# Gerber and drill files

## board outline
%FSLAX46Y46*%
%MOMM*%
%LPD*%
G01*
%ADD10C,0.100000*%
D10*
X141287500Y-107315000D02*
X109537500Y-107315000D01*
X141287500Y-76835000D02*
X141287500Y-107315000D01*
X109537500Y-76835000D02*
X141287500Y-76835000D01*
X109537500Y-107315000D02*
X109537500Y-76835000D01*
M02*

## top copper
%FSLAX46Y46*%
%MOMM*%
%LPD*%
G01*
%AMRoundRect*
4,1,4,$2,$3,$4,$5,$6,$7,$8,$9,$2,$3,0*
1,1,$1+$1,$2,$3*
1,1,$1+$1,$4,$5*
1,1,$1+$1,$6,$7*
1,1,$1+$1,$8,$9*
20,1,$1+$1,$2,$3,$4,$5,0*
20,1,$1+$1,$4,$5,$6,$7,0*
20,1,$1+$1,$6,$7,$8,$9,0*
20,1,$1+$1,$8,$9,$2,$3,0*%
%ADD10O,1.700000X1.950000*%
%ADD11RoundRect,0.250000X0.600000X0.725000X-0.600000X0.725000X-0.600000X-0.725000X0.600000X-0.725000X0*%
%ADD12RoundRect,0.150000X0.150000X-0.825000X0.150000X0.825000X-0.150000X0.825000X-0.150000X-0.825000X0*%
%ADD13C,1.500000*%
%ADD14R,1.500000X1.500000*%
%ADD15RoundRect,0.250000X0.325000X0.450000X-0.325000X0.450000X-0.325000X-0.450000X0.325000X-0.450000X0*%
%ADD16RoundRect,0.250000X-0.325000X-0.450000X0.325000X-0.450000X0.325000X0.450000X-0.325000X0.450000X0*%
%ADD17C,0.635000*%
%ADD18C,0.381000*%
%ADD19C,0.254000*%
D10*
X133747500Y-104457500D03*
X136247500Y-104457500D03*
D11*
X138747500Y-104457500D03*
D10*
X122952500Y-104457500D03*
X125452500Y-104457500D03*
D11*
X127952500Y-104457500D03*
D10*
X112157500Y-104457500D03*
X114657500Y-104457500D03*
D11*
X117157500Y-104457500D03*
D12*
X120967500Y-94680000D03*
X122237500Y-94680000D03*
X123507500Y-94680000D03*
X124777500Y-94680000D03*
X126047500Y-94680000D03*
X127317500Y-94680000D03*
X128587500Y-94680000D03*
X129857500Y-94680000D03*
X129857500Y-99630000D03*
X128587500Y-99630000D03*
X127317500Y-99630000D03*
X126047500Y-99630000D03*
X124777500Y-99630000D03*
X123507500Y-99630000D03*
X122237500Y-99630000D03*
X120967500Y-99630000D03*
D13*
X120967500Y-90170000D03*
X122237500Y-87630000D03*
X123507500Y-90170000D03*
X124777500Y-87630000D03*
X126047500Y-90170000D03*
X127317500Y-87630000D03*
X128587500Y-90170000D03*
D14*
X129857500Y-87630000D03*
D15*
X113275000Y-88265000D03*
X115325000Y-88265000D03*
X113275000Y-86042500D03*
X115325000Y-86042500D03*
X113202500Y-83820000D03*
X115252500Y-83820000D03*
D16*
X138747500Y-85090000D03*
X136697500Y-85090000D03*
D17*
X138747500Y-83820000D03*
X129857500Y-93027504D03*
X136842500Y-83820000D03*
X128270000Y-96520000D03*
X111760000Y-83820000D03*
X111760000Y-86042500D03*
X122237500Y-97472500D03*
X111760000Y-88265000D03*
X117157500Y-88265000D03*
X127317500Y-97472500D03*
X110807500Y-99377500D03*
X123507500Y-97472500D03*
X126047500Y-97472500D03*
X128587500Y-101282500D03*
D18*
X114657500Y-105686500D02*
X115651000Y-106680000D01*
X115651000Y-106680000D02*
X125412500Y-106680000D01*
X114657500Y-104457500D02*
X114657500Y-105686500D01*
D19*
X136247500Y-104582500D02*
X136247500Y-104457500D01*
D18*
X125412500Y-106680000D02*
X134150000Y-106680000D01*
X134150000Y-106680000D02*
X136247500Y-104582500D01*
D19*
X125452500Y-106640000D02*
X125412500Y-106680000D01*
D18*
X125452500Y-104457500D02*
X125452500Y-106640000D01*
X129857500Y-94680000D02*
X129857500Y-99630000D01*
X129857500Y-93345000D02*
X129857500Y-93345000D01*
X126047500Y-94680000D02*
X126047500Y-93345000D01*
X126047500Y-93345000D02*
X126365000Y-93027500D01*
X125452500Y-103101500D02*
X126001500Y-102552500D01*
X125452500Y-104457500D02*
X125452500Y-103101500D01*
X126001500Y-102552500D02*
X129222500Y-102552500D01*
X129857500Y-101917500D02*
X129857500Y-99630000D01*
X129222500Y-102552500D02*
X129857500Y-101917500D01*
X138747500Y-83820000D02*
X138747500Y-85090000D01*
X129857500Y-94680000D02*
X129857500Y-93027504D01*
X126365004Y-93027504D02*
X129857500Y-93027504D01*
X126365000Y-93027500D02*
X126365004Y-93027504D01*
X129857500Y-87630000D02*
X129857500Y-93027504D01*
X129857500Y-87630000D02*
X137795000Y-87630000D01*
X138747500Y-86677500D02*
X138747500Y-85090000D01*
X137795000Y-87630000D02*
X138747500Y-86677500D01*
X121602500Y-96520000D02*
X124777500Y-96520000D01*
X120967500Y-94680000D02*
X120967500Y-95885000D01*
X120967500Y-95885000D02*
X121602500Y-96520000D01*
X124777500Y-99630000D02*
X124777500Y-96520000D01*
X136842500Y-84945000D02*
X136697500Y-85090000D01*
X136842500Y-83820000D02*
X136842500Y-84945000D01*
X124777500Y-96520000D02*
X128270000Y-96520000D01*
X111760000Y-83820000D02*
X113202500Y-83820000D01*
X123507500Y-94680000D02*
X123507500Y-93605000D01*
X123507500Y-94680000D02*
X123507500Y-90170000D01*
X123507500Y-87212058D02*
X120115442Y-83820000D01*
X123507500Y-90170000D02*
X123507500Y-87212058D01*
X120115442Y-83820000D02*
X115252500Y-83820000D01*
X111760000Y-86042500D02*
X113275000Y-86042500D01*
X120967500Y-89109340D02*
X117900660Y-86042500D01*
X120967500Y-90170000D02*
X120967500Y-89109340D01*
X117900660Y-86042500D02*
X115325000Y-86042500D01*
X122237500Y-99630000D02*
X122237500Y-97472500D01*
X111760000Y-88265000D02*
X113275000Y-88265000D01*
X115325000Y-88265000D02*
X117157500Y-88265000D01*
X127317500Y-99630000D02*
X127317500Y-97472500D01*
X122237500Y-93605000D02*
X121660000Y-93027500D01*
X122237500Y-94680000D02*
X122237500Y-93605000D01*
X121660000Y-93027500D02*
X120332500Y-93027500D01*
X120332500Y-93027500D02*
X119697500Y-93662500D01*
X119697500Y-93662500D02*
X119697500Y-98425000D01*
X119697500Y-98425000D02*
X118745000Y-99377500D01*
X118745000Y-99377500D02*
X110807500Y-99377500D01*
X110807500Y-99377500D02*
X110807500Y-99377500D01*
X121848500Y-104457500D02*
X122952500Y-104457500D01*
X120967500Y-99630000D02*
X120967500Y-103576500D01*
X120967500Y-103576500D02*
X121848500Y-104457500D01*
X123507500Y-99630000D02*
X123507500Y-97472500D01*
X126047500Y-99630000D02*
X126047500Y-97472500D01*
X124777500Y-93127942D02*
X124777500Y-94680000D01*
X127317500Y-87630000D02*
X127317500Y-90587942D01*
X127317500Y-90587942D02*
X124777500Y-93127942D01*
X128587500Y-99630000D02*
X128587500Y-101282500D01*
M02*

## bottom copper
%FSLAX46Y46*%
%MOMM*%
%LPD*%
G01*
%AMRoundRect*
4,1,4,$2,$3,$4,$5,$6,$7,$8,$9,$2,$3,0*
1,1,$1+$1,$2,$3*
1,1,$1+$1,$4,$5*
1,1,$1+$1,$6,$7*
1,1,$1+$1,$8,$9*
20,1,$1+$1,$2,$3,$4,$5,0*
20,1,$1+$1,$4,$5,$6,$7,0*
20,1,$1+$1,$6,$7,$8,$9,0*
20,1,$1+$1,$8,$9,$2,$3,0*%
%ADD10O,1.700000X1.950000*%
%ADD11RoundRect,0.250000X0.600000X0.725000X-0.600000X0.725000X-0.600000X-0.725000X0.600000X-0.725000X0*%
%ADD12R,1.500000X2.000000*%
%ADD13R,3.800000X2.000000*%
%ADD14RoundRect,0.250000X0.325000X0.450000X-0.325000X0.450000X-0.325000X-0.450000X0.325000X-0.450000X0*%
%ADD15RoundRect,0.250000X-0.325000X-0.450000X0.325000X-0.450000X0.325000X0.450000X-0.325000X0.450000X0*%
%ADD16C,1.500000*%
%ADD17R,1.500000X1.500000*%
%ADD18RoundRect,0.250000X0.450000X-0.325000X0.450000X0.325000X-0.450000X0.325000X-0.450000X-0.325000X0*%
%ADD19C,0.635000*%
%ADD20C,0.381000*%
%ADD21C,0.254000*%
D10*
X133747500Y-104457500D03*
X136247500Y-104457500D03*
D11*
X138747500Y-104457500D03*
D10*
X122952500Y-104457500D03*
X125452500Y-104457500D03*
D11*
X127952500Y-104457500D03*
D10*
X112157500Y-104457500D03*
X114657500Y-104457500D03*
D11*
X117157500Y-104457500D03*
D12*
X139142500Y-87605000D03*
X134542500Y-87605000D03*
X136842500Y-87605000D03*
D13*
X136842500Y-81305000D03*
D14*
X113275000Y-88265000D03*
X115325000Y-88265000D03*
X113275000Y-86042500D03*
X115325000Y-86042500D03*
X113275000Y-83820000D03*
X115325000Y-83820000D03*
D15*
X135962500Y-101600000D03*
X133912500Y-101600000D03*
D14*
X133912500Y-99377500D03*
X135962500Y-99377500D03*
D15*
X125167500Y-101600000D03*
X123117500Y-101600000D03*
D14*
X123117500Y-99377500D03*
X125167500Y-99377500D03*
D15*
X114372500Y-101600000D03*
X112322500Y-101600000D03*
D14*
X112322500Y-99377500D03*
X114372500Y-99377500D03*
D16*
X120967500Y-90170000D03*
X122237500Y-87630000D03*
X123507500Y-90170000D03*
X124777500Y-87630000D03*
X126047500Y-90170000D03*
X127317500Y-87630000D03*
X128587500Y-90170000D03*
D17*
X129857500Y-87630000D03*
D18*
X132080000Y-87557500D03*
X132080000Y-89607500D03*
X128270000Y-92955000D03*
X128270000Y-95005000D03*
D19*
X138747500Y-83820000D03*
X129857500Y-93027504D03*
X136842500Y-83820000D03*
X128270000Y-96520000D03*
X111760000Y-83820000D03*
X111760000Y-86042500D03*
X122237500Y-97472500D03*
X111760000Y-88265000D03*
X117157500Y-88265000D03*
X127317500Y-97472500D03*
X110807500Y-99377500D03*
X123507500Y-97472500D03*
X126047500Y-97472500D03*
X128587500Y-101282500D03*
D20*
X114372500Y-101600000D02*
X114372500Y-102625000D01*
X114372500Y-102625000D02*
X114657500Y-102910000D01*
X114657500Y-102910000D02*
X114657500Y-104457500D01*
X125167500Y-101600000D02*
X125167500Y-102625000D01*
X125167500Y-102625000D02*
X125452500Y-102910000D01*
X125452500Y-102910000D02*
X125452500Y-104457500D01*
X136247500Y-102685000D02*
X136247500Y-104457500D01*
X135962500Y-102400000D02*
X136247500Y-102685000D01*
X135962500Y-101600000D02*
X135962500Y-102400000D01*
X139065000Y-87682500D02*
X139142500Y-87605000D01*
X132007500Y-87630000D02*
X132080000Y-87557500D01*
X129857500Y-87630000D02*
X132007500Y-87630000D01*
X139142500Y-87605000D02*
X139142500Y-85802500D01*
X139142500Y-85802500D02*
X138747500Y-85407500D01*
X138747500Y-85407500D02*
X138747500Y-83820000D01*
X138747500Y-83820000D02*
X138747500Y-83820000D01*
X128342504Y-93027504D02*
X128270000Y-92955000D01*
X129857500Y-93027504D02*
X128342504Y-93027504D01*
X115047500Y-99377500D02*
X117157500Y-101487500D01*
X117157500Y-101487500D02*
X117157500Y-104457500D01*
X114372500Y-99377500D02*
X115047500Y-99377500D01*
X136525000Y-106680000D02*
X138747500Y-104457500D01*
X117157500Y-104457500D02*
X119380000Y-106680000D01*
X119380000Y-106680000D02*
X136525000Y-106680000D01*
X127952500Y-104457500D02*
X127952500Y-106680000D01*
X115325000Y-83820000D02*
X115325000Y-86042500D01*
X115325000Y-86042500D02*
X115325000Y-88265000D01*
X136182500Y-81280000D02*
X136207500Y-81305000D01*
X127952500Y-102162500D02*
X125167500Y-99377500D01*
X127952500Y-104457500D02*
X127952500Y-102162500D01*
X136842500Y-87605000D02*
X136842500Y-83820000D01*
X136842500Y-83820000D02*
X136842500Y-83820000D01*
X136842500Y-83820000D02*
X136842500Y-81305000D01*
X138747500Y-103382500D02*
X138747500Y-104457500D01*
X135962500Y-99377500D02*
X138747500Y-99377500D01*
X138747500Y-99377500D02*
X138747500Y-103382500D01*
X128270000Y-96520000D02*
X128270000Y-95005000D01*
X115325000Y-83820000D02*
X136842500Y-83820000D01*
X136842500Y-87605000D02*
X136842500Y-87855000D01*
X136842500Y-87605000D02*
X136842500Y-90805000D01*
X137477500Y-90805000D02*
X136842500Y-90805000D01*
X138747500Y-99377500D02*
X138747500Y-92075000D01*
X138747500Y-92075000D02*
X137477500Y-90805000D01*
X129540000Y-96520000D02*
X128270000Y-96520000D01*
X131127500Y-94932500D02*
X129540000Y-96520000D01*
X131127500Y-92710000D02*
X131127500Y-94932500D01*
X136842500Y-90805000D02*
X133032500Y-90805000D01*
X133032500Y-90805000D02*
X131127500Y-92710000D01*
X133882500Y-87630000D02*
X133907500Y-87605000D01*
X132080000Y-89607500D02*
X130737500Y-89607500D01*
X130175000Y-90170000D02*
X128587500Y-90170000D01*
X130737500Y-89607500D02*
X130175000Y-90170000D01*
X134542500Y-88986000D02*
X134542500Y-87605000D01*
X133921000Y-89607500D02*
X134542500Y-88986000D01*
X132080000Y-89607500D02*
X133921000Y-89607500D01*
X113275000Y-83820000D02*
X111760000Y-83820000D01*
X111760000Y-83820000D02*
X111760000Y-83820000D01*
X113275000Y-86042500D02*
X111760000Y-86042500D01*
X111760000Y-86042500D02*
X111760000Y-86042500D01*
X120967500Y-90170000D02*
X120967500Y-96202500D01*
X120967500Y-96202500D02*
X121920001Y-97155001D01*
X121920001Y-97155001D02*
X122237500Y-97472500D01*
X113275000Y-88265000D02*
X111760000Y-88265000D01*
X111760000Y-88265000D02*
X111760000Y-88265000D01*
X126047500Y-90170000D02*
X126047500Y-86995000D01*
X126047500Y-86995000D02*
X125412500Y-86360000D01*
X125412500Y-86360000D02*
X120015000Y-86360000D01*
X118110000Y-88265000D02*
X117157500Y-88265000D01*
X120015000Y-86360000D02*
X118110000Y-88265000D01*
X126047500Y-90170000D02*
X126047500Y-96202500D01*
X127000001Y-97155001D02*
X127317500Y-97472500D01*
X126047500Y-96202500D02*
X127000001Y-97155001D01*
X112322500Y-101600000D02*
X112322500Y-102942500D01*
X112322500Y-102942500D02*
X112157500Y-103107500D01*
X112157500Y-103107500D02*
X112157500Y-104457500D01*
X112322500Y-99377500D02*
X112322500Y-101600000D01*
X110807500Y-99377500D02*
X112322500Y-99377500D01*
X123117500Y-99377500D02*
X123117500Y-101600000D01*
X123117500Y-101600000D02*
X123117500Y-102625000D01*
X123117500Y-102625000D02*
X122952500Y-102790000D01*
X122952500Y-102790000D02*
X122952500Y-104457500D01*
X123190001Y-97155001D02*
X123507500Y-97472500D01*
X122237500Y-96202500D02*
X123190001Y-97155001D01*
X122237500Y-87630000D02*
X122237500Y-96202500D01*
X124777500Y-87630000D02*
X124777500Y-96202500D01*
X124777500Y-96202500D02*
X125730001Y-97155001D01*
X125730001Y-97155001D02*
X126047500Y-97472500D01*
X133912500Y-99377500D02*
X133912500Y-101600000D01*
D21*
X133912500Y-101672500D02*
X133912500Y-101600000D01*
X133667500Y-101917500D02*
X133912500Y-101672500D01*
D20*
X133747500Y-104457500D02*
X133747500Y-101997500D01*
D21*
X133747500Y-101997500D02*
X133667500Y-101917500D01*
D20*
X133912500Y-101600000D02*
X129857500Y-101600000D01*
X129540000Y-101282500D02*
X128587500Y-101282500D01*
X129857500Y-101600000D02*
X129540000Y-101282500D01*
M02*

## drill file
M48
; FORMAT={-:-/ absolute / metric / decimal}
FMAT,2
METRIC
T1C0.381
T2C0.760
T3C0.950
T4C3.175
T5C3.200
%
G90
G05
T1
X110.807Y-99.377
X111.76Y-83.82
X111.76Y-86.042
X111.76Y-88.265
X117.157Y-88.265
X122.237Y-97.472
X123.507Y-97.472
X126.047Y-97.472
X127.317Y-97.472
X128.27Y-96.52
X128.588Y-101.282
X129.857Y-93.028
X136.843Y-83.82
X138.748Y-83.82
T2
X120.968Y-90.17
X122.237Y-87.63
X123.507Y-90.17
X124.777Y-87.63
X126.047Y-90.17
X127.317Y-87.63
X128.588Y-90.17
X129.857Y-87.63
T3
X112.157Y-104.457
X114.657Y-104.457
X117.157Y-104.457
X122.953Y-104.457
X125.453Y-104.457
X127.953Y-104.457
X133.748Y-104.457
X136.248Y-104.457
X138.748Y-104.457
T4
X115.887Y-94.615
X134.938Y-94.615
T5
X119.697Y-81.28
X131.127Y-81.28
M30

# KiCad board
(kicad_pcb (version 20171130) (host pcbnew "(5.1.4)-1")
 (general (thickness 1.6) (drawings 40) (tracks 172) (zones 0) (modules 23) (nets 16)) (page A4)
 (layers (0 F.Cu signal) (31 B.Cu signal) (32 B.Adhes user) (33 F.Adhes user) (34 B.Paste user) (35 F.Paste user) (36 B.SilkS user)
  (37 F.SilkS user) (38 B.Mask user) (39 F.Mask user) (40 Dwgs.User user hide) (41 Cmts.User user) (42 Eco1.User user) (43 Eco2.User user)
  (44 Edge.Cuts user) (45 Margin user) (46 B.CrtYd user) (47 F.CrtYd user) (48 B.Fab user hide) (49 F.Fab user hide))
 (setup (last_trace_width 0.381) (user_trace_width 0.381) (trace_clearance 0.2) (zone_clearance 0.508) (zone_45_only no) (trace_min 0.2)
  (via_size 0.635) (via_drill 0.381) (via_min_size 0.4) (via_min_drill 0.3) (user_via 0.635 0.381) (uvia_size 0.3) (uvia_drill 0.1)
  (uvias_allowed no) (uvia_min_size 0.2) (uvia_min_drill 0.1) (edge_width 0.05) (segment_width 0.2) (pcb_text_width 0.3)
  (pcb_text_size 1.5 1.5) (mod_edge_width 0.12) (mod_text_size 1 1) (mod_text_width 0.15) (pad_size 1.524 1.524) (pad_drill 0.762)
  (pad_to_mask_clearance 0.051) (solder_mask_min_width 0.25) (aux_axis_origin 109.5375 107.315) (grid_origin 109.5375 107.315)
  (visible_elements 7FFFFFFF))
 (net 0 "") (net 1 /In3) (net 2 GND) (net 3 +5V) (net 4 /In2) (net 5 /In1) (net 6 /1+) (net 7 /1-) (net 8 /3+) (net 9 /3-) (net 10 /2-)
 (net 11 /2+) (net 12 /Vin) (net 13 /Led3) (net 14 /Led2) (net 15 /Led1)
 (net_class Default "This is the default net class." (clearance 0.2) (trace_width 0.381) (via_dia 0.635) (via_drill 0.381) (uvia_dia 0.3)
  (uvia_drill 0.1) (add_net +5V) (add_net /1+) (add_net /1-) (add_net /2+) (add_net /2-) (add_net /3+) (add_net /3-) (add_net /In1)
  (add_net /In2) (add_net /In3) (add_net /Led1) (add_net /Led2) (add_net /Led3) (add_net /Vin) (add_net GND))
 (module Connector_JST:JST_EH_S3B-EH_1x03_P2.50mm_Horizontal (layer F.Cu) (at 138.7475 104.4575 180)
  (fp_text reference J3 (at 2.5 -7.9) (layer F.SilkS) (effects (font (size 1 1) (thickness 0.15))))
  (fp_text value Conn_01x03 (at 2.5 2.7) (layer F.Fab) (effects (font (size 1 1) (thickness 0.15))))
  (pad 3 thru_hole oval (at 5 0 180) (size 1.7 1.95) (drill 0.95) (layers *.Cu *.Mask) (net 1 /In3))
  (pad 2 thru_hole oval (at 2.5 0 180) (size 1.7 1.95) (drill 0.95) (layers *.Cu *.Mask) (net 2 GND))
  (pad 1 thru_hole roundrect (at 0 0 180) (size 1.7 1.95) (drill 0.95) (layers *.Cu *.Mask) (roundrect_rratio 0.147059) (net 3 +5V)))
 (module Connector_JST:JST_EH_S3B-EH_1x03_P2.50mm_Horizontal (layer F.Cu) (at 127.9525 104.4575 180)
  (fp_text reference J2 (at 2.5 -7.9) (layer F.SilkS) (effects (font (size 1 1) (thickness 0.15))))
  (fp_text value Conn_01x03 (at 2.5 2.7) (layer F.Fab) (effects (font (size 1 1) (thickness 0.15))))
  (pad 3 thru_hole oval (at 5 0 180) (size 1.7 1.95) (drill 0.95) (layers *.Cu *.Mask) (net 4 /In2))
  (pad 2 thru_hole oval (at 2.5 0 180) (size 1.7 1.95) (drill 0.95) (layers *.Cu *.Mask) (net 2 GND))
  (pad 1 thru_hole roundrect (at 0 0 180) (size 1.7 1.95) (drill 0.95) (layers *.Cu *.Mask) (roundrect_rratio 0.147059) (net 3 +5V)))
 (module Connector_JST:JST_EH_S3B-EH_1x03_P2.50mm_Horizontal (layer F.Cu) (at 117.1575 104.4575 180)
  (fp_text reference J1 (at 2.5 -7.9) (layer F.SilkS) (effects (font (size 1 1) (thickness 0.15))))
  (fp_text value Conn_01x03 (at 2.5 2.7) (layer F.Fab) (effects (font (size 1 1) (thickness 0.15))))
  (pad 3 thru_hole oval (at 5 0 180) (size 1.7 1.95) (drill 0.95) (layers *.Cu *.Mask) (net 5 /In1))
  (pad 2 thru_hole oval (at 2.5 0 180) (size 1.7 1.95) (drill 0.95) (layers *.Cu *.Mask) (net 2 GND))
  (pad 1 thru_hole roundrect (at 0 0 180) (size 1.7 1.95) (drill 0.95) (layers *.Cu *.Mask) (roundrect_rratio 0.147059) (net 3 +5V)))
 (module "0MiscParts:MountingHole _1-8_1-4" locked (layer F.Cu) (at 134.9375 94.615)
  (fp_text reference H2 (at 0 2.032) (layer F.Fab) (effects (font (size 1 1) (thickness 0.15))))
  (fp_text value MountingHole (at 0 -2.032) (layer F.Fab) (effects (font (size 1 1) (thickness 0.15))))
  (pad "" np_thru_hole circle (at 0 0) (size 3.175 3.175) (drill 3.175) (layers *.Cu *.Mask)))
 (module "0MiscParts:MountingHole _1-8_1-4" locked (layer F.Cu) (at 115.8875 94.615)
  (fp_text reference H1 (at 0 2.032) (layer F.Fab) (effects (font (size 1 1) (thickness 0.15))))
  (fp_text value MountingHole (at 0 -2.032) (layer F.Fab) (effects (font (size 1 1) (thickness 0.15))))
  (pad "" np_thru_hole circle (at 0 0) (size 3.175 3.175) (drill 3.175) (layers *.Cu *.Mask)))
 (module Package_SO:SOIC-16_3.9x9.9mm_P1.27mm (layer F.Cu) (at 125.4125 97.155 90)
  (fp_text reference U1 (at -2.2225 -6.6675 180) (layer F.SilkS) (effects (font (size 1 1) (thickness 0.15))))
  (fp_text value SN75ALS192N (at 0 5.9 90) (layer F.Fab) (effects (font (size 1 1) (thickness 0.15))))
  (pad 16 smd roundrect (at 2.475 -4.445 90) (size 1.95 0.6) (layers F.Cu F.Paste F.Mask) (roundrect_rratio 0.25) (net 3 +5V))
  (pad 15 smd roundrect (at 2.475 -3.175 90) (size 1.95 0.6) (layers F.Cu F.Paste F.Mask) (roundrect_rratio 0.25) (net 5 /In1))
  (pad 14 smd roundrect (at 2.475 -1.905 90) (size 1.95 0.6) (layers F.Cu F.Paste F.Mask) (roundrect_rratio 0.25) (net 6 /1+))
  (pad 13 smd roundrect (at 2.475 -0.635 90) (size 1.95 0.6) (layers F.Cu F.Paste F.Mask) (roundrect_rratio 0.25) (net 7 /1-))
  (pad 12 smd roundrect (at 2.475 0.635 90) (size 1.95 0.6) (layers F.Cu F.Paste F.Mask) (roundrect_rratio 0.25) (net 2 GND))
  (pad 11 smd roundrect (at 2.475 1.905 90) (size 1.95 0.6) (layers F.Cu F.Paste F.Mask) (roundrect_rratio 0.25))
  (pad 10 smd roundrect (at 2.475 3.175 90) (size 1.95 0.6) (layers F.Cu F.Paste F.Mask) (roundrect_rratio 0.25))
  (pad 9 smd roundrect (at 2.475 4.445 90) (size 1.95 0.6) (layers F.Cu F.Paste F.Mask) (roundrect_rratio 0.25) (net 2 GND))
  (pad 8 smd roundrect (at -2.475 4.445 90) (size 1.95 0.6) (layers F.Cu F.Paste F.Mask) (roundrect_rratio 0.25) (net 2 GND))
  (pad 7 smd roundrect (at -2.475 3.175 90) (size 1.95 0.6) (layers F.Cu F.Paste F.Mask) (roundrect_rratio 0.25) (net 1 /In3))
  (pad 6 smd roundrect (at -2.475 1.905 90) (size 1.95 0.6) (layers F.Cu F.Paste F.Mask) (roundrect_rratio 0.25) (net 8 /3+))
  (pad 5 smd roundrect (at -2.475 0.635 90) (size 1.95 0.6) (layers F.Cu F.Paste F.Mask) (roundrect_rratio 0.25) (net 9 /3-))
  (pad 4 smd roundrect (at -2.475 -0.635 90) (size 1.95 0.6) (layers F.Cu F.Paste F.Mask) (roundrect_rratio 0.25) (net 3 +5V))
  (pad 3 smd roundrect (at -2.475 -1.905 90) (size 1.95 0.6) (layers F.Cu F.Paste F.Mask) (roundrect_rratio 0.25) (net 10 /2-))
  (pad 2 smd roundrect (at -2.475 -3.175 90) (size 1.95 0.6) (layers F.Cu F.Paste F.Mask) (roundrect_rratio 0.25) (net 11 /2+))
  (pad 1 smd roundrect (at -2.475 -4.445 90) (size 1.95 0.6) (layers F.Cu F.Paste F.Mask) (roundrect_rratio 0.25) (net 4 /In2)))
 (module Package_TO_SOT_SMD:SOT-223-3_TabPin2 (layer B.Cu) (at 136.8425 84.455 90)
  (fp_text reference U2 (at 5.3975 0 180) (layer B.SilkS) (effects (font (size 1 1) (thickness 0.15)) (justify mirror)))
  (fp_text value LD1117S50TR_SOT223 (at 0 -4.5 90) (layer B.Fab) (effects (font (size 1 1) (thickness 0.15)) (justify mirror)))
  (pad 1 smd rect (at -3.15 2.3 90) (size 2 1.5) (layers B.Cu B.Paste B.Mask) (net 2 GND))
  (pad 3 smd rect (at -3.15 -2.3 90) (size 2 1.5) (layers B.Cu B.Paste B.Mask) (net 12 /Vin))
  (pad 2 smd rect (at -3.15 0 90) (size 2 1.5) (layers B.Cu B.Paste B.Mask) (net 3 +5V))
  (pad 2 smd rect (at 3.15 0 90) (size 2 3.8) (layers B.Cu B.Paste B.Mask) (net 3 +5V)))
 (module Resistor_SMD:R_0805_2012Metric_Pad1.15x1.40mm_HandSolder (layer B.Cu) (at 114.3 88.265 180)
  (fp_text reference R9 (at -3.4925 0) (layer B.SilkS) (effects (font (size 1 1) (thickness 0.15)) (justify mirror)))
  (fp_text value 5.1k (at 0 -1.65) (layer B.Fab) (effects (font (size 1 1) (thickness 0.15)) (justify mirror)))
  (pad 2 smd roundrect (at 1.025 0 180) (size 1.15 1.4) (layers B.Cu B.Paste B.Mask) (roundrect_rratio 0.217391) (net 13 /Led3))
  (pad 1 smd roundrect (at -1.025 0 180) (size 1.15 1.4) (layers B.Cu B.Paste B.Mask) (roundrect_rratio 0.217391) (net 3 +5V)))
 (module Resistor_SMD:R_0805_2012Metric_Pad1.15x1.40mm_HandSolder (layer B.Cu) (at 114.3 86.0425 180)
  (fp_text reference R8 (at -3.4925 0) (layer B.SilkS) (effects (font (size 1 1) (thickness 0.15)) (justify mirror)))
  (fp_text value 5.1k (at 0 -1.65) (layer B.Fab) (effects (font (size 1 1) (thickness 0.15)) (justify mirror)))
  (pad 2 smd roundrect (at 1.025 0 180) (size 1.15 1.4) (layers B.Cu B.Paste B.Mask) (roundrect_rratio 0.217391) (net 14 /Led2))
  (pad 1 smd roundrect (at -1.025 0 180) (size 1.15 1.4) (layers B.Cu B.Paste B.Mask) (roundrect_rratio 0.217391) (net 3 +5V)))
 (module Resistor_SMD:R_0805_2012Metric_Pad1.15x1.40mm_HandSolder (layer B.Cu) (at 114.3 83.82 180)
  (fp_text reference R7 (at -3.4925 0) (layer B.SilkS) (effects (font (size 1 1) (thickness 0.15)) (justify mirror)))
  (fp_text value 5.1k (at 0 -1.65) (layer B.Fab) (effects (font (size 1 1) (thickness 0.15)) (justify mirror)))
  (pad 2 smd roundrect (at 1.025 0 180) (size 1.15 1.4) (layers B.Cu B.Paste B.Mask) (roundrect_rratio 0.217391) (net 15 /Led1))
  (pad 1 smd roundrect (at -1.025 0 180) (size 1.15 1.4) (layers B.Cu B.Paste B.Mask) (roundrect_rratio 0.217391) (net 3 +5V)))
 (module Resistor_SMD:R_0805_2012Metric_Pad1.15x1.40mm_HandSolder (layer B.Cu) (at 134.9375 101.6)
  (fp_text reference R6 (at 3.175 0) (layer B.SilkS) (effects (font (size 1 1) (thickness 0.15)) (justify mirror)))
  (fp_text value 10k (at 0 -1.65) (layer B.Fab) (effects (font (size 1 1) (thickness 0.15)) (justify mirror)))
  (pad 2 smd roundrect (at 1.025 0) (size 1.15 1.4) (layers B.Cu B.Paste B.Mask) (roundrect_rratio 0.217391) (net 2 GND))
  (pad 1 smd roundrect (at -1.025 0) (size 1.15 1.4) (layers B.Cu B.Paste B.Mask) (roundrect_rratio 0.217391) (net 1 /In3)))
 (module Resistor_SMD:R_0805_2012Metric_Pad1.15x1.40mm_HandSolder (layer B.Cu) (at 134.9375 99.3775 180)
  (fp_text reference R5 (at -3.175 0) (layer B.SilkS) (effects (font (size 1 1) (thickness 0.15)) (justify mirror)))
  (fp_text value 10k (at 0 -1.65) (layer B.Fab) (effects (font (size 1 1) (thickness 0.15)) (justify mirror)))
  (pad 2 smd roundrect (at 1.025 0 180) (size 1.15 1.4) (layers B.Cu B.Paste B.Mask) (roundrect_rratio 0.217391) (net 1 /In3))
  (pad 1 smd roundrect (at -1.025 0 180) (size 1.15 1.4) (layers B.Cu B.Paste B.Mask) (roundrect_rratio 0.217391) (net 3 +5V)))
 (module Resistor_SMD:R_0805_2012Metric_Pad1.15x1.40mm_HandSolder (layer B.Cu) (at 124.1425 101.6)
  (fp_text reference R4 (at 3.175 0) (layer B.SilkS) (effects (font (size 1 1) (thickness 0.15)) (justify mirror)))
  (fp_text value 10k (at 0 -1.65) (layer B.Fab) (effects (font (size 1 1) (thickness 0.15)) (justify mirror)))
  (pad 2 smd roundrect (at 1.025 0) (size 1.15 1.4) (layers B.Cu B.Paste B.Mask) (roundrect_rratio 0.217391) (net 2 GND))
  (pad 1 smd roundrect (at -1.025 0) (size 1.15 1.4) (layers B.Cu B.Paste B.Mask) (roundrect_rratio 0.217391) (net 4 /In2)))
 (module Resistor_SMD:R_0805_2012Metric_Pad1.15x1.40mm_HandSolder (layer B.Cu) (at 124.1425 99.3775 180)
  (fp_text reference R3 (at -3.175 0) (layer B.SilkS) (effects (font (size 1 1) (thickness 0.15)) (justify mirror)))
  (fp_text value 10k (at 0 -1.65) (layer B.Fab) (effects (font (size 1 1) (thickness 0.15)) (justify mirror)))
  (pad 2 smd roundrect (at 1.025 0 180) (size 1.15 1.4) (layers B.Cu B.Paste B.Mask) (roundrect_rratio 0.217391) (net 4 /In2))
  (pad 1 smd roundrect (at -1.025 0 180) (size 1.15 1.4) (layers B.Cu B.Paste B.Mask) (roundrect_rratio 0.217391) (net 3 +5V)))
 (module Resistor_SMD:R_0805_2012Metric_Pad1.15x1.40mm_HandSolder (layer B.Cu) (at 113.3475 101.6)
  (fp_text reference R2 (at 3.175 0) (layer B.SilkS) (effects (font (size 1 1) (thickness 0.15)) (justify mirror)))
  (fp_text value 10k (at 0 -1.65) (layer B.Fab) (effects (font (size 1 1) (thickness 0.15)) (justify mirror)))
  (pad 2 smd roundrect (at 1.025 0) (size 1.15 1.4) (layers B.Cu B.Paste B.Mask) (roundrect_rratio 0.217391) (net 2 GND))
  (pad 1 smd roundrect (at -1.025 0) (size 1.15 1.4) (layers B.Cu B.Paste B.Mask) (roundrect_rratio 0.217391) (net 5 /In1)))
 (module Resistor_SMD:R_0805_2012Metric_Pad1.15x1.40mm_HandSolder (layer B.Cu) (at 113.3475 99.3775 180)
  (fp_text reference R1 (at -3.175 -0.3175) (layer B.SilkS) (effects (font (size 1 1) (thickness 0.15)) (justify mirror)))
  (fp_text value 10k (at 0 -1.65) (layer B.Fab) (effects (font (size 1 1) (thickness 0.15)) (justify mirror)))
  (pad 2 smd roundrect (at 1.025 0 180) (size 1.15 1.4) (layers B.Cu B.Paste B.Mask) (roundrect_rratio 0.217391) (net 5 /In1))
  (pad 1 smd roundrect (at -1.025 0 180) (size 1.15 1.4) (layers B.Cu B.Paste B.Mask) (roundrect_rratio 0.217391) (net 3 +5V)))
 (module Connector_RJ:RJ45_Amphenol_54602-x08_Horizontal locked (layer F.Cu) (at 129.8575 87.63 180)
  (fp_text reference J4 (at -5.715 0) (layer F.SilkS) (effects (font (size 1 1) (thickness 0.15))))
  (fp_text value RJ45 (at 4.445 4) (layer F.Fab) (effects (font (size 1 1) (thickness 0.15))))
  (pad 8 thru_hole circle (at 8.89 -2.54 180) (size 1.5 1.5) (drill 0.76) (layers *.Cu *.Mask) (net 11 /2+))
  (pad 7 thru_hole circle (at 7.62 0 180) (size 1.5 1.5) (drill 0.76) (layers *.Cu *.Mask) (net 10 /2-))
  (pad 6 thru_hole circle (at 6.35 -2.54 180) (size 1.5 1.5) (drill 0.76) (layers *.Cu *.Mask) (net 6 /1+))
  (pad 5 thru_hole circle (at 5.08 0 180) (size 1.5 1.5) (drill 0.76) (layers *.Cu *.Mask) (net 9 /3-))
  (pad 4 thru_hole circle (at 3.81 -2.54 180) (size 1.5 1.5) (drill 0.76) (layers *.Cu *.Mask) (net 8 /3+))
  (pad 3 thru_hole circle (at 2.54 0 180) (size 1.5 1.5) (drill 0.76) (layers *.Cu *.Mask) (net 7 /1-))
  (pad 2 thru_hole circle (at 1.27 -2.54 180) (size 1.5 1.5) (drill 0.76) (layers *.Cu *.Mask) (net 12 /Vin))
  (pad 1 thru_hole rect (at 0 0 180) (size 1.5 1.5) (drill 0.76) (layers *.Cu *.Mask) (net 2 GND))
  (pad "" np_thru_hole circle (at -1.27 6.35 180) (size 3.2 3.2) (drill 3.2) (layers *.Cu *.Mask))
  (pad "" np_thru_hole circle (at 10.16 6.35 180) (size 3.2 3.2) (drill 3.2) (layers *.Cu *.Mask)))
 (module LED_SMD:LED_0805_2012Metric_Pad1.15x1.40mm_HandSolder (layer F.Cu) (at 114.3 88.265 180)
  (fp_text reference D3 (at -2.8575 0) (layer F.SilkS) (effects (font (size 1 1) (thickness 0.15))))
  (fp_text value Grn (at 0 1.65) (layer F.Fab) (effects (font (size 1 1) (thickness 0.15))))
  (pad 2 smd roundrect (at 1.025 0 180) (size 1.15 1.4) (layers F.Cu F.Paste F.Mask) (roundrect_rratio 0.217391) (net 13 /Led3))
  (pad 1 smd roundrect (at -1.025 0 180) (size 1.15 1.4) (layers F.Cu F.Paste F.Mask) (roundrect_rratio 0.217391) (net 8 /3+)))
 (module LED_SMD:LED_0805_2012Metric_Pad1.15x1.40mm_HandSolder (layer F.Cu) (at 114.3 86.0425 180)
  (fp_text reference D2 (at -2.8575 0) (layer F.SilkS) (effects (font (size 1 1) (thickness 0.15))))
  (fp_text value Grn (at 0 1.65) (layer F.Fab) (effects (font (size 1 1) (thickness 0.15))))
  (pad 2 smd roundrect (at 1.025 0 180) (size 1.15 1.4) (layers F.Cu F.Paste F.Mask) (roundrect_rratio 0.217391) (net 14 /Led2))
  (pad 1 smd roundrect (at -1.025 0 180) (size 1.15 1.4) (layers F.Cu F.Paste F.Mask) (roundrect_rratio 0.217391) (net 11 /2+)))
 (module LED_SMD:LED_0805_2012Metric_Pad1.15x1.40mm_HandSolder (layer F.Cu) (at 114.2275 83.82 180)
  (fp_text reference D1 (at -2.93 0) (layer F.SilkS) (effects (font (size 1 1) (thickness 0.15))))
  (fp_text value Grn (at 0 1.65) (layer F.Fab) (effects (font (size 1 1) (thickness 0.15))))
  (pad 2 smd roundrect (at 1.025 0 180) (size 1.15 1.4) (layers F.Cu F.Paste F.Mask) (roundrect_rratio 0.217391) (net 15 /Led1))
  (pad 1 smd roundrect (at -1.025 0 180) (size 1.15 1.4) (layers F.Cu F.Paste F.Mask) (roundrect_rratio 0.217391) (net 6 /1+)))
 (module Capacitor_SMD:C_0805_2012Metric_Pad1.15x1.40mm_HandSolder (layer F.Cu) (at 137.7225 85.09)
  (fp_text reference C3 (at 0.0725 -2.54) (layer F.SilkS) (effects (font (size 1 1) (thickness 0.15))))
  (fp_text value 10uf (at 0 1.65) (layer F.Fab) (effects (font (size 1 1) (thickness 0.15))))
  (pad 2 smd roundrect (at 1.025 0) (size 1.15 1.4) (layers F.Cu F.Paste F.Mask) (roundrect_rratio 0.217391) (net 2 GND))
  (pad 1 smd roundrect (at -1.025 0) (size 1.15 1.4) (layers F.Cu F.Paste F.Mask) (roundrect_rratio 0.217391) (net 3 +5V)))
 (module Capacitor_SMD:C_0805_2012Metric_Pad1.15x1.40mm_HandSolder (layer B.Cu) (at 132.08 88.5825 90)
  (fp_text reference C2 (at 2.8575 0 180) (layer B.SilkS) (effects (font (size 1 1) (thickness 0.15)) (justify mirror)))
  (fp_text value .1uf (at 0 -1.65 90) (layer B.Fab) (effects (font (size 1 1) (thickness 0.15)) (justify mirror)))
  (pad 2 smd roundrect (at 1.025 0 90) (size 1.15 1.4) (layers B.Cu B.Paste B.Mask) (roundrect_rratio 0.217391) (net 2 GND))
  (pad 1 smd roundrect (at -1.025 0 90) (size 1.15 1.4) (layers B.Cu B.Paste B.Mask) (roundrect_rratio 0.217391) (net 12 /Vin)))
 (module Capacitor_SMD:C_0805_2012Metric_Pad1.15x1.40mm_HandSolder (layer B.Cu) (at 128.27 93.98 90)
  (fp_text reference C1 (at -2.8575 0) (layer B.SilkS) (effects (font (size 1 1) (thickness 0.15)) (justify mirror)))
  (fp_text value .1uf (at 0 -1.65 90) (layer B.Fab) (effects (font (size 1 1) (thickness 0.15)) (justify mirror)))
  (pad 2 smd roundrect (at 1.025 0 90) (size 1.15 1.4) (layers B.Cu B.Paste B.Mask) (roundrect_rratio 0.217391) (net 2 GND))
  (pad 1 smd roundrect (at -1.025 0 90) (size 1.15 1.4) (layers B.Cu B.Paste B.Mask) (roundrect_rratio 0.217391) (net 3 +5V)))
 (gr_line (start 141.2875 107.315) (end 109.5375 107.315) (layer Edge.Cuts) (width 0.1))
 (gr_line (start 141.2875 76.835) (end 141.2875 107.315) (layer Edge.Cuts) (width 0.1))
 (gr_line (start 109.5375 76.835) (end 141.2875 76.835) (layer Edge.Cuts) (width 0.1))
 (gr_line (start 109.5375 107.315) (end 109.5375 76.835) (layer Edge.Cuts) (width 0.1))
 (segment (start 114.3725 101.6) (end 114.3725 102.625) (width 0.381) (layer B.Cu) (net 2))
 (segment (start 114.3725 102.625) (end 114.6575 102.91) (width 0.381) (layer B.Cu) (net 2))
 (segment (start 114.6575 102.91) (end 114.6575 104.4575) (width 0.381) (layer B.Cu) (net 2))
 (segment (start 125.1675 101.6) (end 125.1675 102.625) (width 0.381) (layer B.Cu) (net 2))
 (segment (start 125.1675 102.625) (end 125.4525 102.91) (width 0.381) (layer B.Cu) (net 2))
 (segment (start 125.4525 102.91) (end 125.4525 104.4575) (width 0.381) (layer B.Cu) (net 2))
 (segment (start 136.2475 102.685) (end 136.2475 104.4575) (width 0.381) (layer B.Cu) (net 2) (status 1000000))
 (segment (start 135.9625 102.4) (end 136.2475 102.685) (width 0.381) (layer B.Cu) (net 2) (status 1000000))
 (segment (start 135.9625 101.6) (end 135.9625 102.4) (width 0.381) (layer B.Cu) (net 2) (status 1000000))
 (segment (start 114.6575 105.6865) (end 115.651 106.68) (width 0.381) (layer F.Cu) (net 2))
 (segment (start 115.651 106.68) (end 125.4125 106.68) (width 0.381) (layer F.Cu) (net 2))
 (segment (start 114.6575 104.4575) (end 114.6575 105.6865) (width 0.381) (layer F.Cu) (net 2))
 (segment (start 136.2475 104.5825) (end 136.2475 104.4575) (width 0.254) (layer F.Cu) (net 2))
 (segment (start 125.4125 106.68) (end 134.15 106.68) (width 0.381) (layer F.Cu) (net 2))
 (segment (start 134.15 106.68) (end 136.2475 104.5825) (width 0.381) (layer F.Cu) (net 2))
 (segment (start 125.4525 106.64) (end 125.4125 106.68) (width 0.254) (layer F.Cu) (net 2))
 (segment (start 125.4525 104.4575) (end 125.4525 106.64) (width 0.381) (layer F.Cu) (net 2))
 (segment (start 129.8575 94.68) (end 129.8575 99.63) (width 0.381) (layer F.Cu) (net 2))
 (segment (start 129.8575 93.345) (end 129.8575 93.345) (width 0.381) (layer F.Cu) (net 2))
 (segment (start 126.0475 94.68) (end 126.0475 93.345) (width 0.381) (layer F.Cu) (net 2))
 (segment (start 126.0475 93.345) (end 126.365 93.0275) (width 0.381) (layer F.Cu) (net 2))
 (segment (start 125.4525 103.1015) (end 126.0015 102.5525) (width 0.381) (layer F.Cu) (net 2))
 (segment (start 125.4525 104.4575) (end 125.4525 103.1015) (width 0.381) (layer F.Cu) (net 2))
 (segment (start 126.0015 102.5525) (end 129.2225 102.5525) (width 0.381) (layer F.Cu) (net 2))
 (segment (start 129.8575 101.9175) (end 129.8575 99.63) (width 0.381) (layer F.Cu) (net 2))
 (segment (start 129.2225 102.5525) (end 129.8575 101.9175) (width 0.381) (layer F.Cu) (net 2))
 (segment (start 139.065 87.6825) (end 139.1425 87.605) (width 0.381) (layer B.Cu) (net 2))
 (segment (start 132.0075 87.63) (end 132.08 87.5575) (width 0.381) (layer B.Cu) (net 2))
 (segment (start 129.8575 87.63) (end 132.0075 87.63) (width 0.381) (layer B.Cu) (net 2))
 (segment (start 139.1425 87.605) (end 139.1425 85.8025) (width 0.381) (layer B.Cu) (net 2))
 (segment (start 139.1425 85.8025) (end 138.7475 85.4075) (width 0.381) (layer B.Cu) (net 2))
 (segment (start 138.7475 85.4075) (end 138.7475 83.82) (width 0.381) (layer B.Cu) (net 2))
 (segment (start 138.7475 83.82) (end 138.7475 83.82) (width 0.381) (layer B.Cu) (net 2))
 (via (at 138.7475 83.82) (size 0.635) (drill 0.381) (layers F.Cu B.Cu) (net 2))
 (segment (start 138.7475 83.82) (end 138.7475 85.09) (width 0.381) (layer F.Cu) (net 2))
 (via (at 129.8575 93.027504) (size 0.635) (drill 0.381) (layers F.Cu B.Cu) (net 2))
 (segment (start 129.8575 94.68) (end 129.8575 93.027504) (width 0.381) (layer F.Cu) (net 2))
 (segment (start 126.365004 93.027504) (end 129.8575 93.027504) (width 0.381) (layer F.Cu) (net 2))
 (segment (start 126.365 93.0275) (end 126.365004 93.027504) (width 0.381) (layer F.Cu) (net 2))
 (segment (start 129.8575 87.63) (end 129.8575 93.027504) (width 0.381) (layer F.Cu) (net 2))
 (segment (start 128.342504 93.027504) (end 128.27 92.955) (width 0.381) (layer B.Cu) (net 2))
 (segment (start 129.8575 93.027504) (end 128.342504 93.027504) (width 0.381) (layer B.Cu) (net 2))
 (segment (start 129.8575 87.63) (end 137.795 87.63) (width 0.381) (layer F.Cu) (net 2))
 (segment (start 138.7475 86.6775) (end 138.7475 85.09) (width 0.381) (layer F.Cu) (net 2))
 (segment (start 137.795 87.63) (end 138.7475 86.6775) (width 0.381) (layer F.Cu) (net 2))
 (segment (start 115.0475 99.3775) (end 117.1575 101.4875) (width 0.381) (layer B.Cu) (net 3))
 (segment (start 117.1575 101.4875) (end 117.1575 104.4575) (width 0.381) (layer B.Cu) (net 3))
 (segment (start 114.3725 99.3775) (end 115.0475 99.3775) (width 0.381) (layer B.Cu) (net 3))
 (segment (start 136.525 106.68) (end 138.7475 104.4575) (width 0.381) (layer B.Cu) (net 3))
 (segment (start 117.1575 104.4575) (end 119.38 106.68) (width 0.381) (layer B.Cu) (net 3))
 (segment (start 119.38 106.68) (end 136.525 106.68) (width 0.381) (layer B.Cu) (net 3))
 (segment (start 127.9525 104.4575) (end 127.9525 106.68) (width 0.381) (layer B.Cu) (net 3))
 (segment (start 115.325 83.82) (end 115.325 86.0425) (width 0.381) (layer B.Cu) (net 3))
 (segment (start 115.325 86.0425) (end 115.325 88.265) (width 0.381) (layer B.Cu) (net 3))
 (segment (start 136.1825 81.28) (end 136.2075 81.305) (width 0.381) (layer B.Cu) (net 3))
 (segment (start 121.6025 96.52) (end 124.7775 96.52) (width 0.381) (layer F.Cu) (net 3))
 (segment (start 120.9675 94.68) (end 120.9675 95.885) (width 0.381) (layer F.Cu) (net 3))
 (segment (start 120.9675 95.885) (end 121.6025 96.52) (width 0.381) (layer F.Cu) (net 3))
 (segment (start 127.9525 102.1625) (end 125.1675 99.3775) (width 0.381) (layer B.Cu) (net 3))
 (segment (start 127.9525 104.4575) (end 127.9525 102.1625) (width 0.381) (layer B.Cu) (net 3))
 (segment (start 124.7775 99.63) (end 124.7775 96.52) (width 0.381) (layer F.Cu) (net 3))
 (segment (start 136.8425 87.605) (end 136.8425 83.82) (width 0.381) (layer B.Cu) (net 3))
 (segment (start 136.8425 83.82) (end 136.8425 83.82) (width 0.381) (layer B.Cu) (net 3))
 (segment (start 136.8425 83.82) (end 136.8425 81.305) (width 0.381) (layer B.Cu) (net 3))
 (via (at 136.8425 83.82) (size 0.635) (drill 0.381) (layers F.Cu B.Cu) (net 3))
 (segment (start 136.8425 84.945) (end 136.6975 85.09) (width 0.381) (layer F.Cu) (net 3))
 (segment (start 136.8425 83.82) (end 136.8425 84.945) (width 0.381) (layer F.Cu) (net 3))
 (segment (start 138.7475 103.3825) (end 138.7475 104.4575) (width 0.381) (layer B.Cu) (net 3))
 (segment (start 135.9625 99.3775) (end 138.7475 99.3775) (width 0.381) (layer B.Cu) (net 3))
 (segment (start 138.7475 99.3775) (end 138.7475 103.3825) (width 0.381) (layer B.Cu) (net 3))
 (segment (start 124.7775 96.52) (end 128.27 96.52) (width 0.381) (layer F.Cu) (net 3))
 (via (at 128.27 96.52) (size 0.635) (drill 0.381) (layers F.Cu B.Cu) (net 3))
 (segment (start 128.27 96.52) (end 128.27 95.005) (width 0.381) (layer B.Cu) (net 3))
 (segment (start 115.325 83.82) (end 136.8425 83.82) (width 0.381) (layer B.Cu) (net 3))
 (segment (start 136.8425 87.605) (end 136.8425 87.855) (width 0.381) (layer B.Cu) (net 3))
 (segment (start 136.8425 87.605) (end 136.8425 90.805) (width 0.381) (layer B.Cu) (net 3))
 (segment (start 137.4775 90.805) (end 136.8425 90.805) (width 0.381) (layer B.Cu) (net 3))
 (segment (start 138.7475 99.3775) (end 138.7475 92.075) (width 0.381) (layer B.Cu) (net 3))
 (segment (start 138.7475 92.075) (end 137.4775 90.805) (width 0.381) (layer B.Cu) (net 3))
 (segment (start 129.54 96.52) (end 128.27 96.52) (width 0.381) (layer B.Cu) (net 3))
 (segment (start 131.1275 94.9325) (end 129.54 96.52) (width 0.381) (layer B.Cu) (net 3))
 (segment (start 131.1275 92.71) (end 131.1275 94.9325) (width 0.381) (layer B.Cu) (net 3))
 (segment (start 136.8425 90.805) (end 133.0325 90.805) (width 0.381) (layer B.Cu) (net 3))
 (segment (start 133.0325 90.805) (end 131.1275 92.71) (width 0.381) (layer B.Cu) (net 3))
 (segment (start 133.8825 87.63) (end 133.9075 87.605) (width 0.381) (layer B.Cu) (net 12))
 (segment (start 132.08 89.6075) (end 130.7375 89.6075) (width 0.381) (layer B.Cu) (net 12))
 (segment (start 130.175 90.17) (end 128.5875 90.17) (width 0.381) (layer B.Cu) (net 12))
 (segment (start 130.7375 89.6075) (end 130.175 90.17) (width 0.381) (layer B.Cu) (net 12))
 (segment (start 134.5425 88.986) (end 134.5425 87.605) (width 0.381) (layer B.Cu) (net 12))
 (segment (start 133.921 89.6075) (end 134.5425 88.986) (width 0.381) (layer B.Cu) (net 12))
 (segment (start 132.08 89.6075) (end 133.921 89.6075) (width 0.381) (layer B.Cu) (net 12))
 (segment (start 113.275 83.82) (end 111.76 83.82) (width 0.381) (layer B.Cu) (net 15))
 (segment (start 111.76 83.82) (end 111.76 83.82) (width 0.381) (layer B.Cu) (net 15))
 (via (at 111.76 83.82) (size 0.635) (drill 0.381) (layers F.Cu B.Cu) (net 15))
 (segment (start 111.76 83.82) (end 113.2025 83.82) (width 0.381) (layer F.Cu) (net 15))
 (segment (start 123.5075 94.68) (end 123.5075 93.605) (width 0.381) (layer F.Cu) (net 6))
 (segment (start 123.5075 94.68) (end 123.5075 90.17) (width 0.381) (layer F.Cu) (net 6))
 (segment (start 123.5075 87.212058) (end 120.115442 83.82) (width 0.381) (layer F.Cu) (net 6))
 (segment (start 123.5075 90.17) (end 123.5075 87.212058) (width 0.381) (layer F.Cu) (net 6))
 (segment (start 120.115442 83.82) (end 115.2525 83.82) (width 0.381) (layer F.Cu) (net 6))
 (segment (start 113.275 86.0425) (end 111.76 86.0425) (width 0.381) (layer B.Cu) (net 14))
 (segment (start 111.76 86.0425) (end 111.76 86.0425) (width 0.381) (layer B.Cu) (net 14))
 (via (at 111.76 86.0425) (size 0.635) (drill 0.381) (layers F.Cu B.Cu) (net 14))
 (segment (start 111.76 86.0425) (end 113.275 86.0425) (width 0.381) (layer F.Cu) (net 14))
 (segment (start 120.9675 89.10934) (end 117.90066 86.0425) (width 0.381) (layer F.Cu) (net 11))
 (segment (start 120.9675 90.17) (end 120.9675 89.10934) (width 0.381) (layer F.Cu) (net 11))
 (segment (start 117.90066 86.0425) (end 115.325 86.0425) (width 0.381) (layer F.Cu) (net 11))
 (via (at 122.2375 97.4725) (size 0.635) (drill 0.381) (layers F.Cu B.Cu) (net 11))
 (segment (start 122.2375 99.63) (end 122.2375 97.4725) (width 0.381) (layer F.Cu) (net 11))
 (segment (start 120.9675 90.17) (end 120.9675 96.2025) (width 0.381) (layer B.Cu) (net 11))
 (segment (start 120.9675 96.2025) (end 121.920001 97.155001) (width 0.381) (layer B.Cu) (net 11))
 (segment (start 121.920001 97.155001) (end 122.2375 97.4725) (width 0.381) (layer B.Cu) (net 11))
 (segment (start 113.275 88.265) (end 111.76 88.265) (width 0.381) (layer B.Cu) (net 13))
 (segment (start 111.76 88.265) (end 111.76 88.265) (width 0.381) (layer B.Cu) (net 13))
 (via (at 111.76 88.265) (size 0.635) (drill 0.381) (layers F.Cu B.Cu) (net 13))
 (segment (start 111.76 88.265) (end 113.275 88.265) (width 0.381) (layer F.Cu) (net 13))
 (via (at 117.1575 88.265) (size 0.635) (drill 0.381) (layers F.Cu B.Cu) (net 8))
 (segment (start 126.0475 90.17) (end 126.0475 86.995) (width 0.381) (layer B.Cu) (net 8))
 (segment (start 126.0475 86.995) (end 125.4125 86.36) (width 0.381) (layer B.Cu) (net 8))
 (segment (start 125.4125 86.36) (end 120.015 86.36) (width 0.381) (layer B.Cu) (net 8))
 (segment (start 118.11 88.265) (end 117.1575 88.265) (width 0.381) (layer B.Cu) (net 8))
 (segment (start 120.015 86.36) (end 118.11 88.265) (width 0.381) (layer B.Cu) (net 8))
 (segment (start 115.325 88.265) (end 117.1575 88.265) (width 0.381) (layer F.Cu) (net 8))
 (via (at 127.3175 97.4725) (size 0.635) (drill 0.381) (layers F.Cu B.Cu) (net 8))
 (segment (start 127.3175 99.63) (end 127.3175 97.4725) (width 0.381) (layer F.Cu) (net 8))
 (segment (start 126.0475 90.17) (end 126.0475 96.2025) (width 0.381) (layer B.Cu) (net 8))
 (segment (start 127.000001 97.155001) (end 127.3175 97.4725) (width 0.381) (layer B.Cu) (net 8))
 (segment (start 126.0475 96.2025) (end 127.000001 97.155001) (width 0.381) (layer B.Cu) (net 8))
 (segment (start 112.3225 101.6) (end 112.3225 102.9425) (width 0.381) (layer B.Cu) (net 5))
 (segment (start 112.3225 102.9425) (end 112.1575 103.1075) (width 0.381) (layer B.Cu) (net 5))
 (segment (start 112.1575 103.1075) (end 112.1575 104.4575) (width 0.381) (layer B.Cu) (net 5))
 (segment (start 112.3225 99.3775) (end 112.3225 101.6) (width 0.381) (layer B.Cu) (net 5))
 (segment (start 122.2375 93.605) (end 121.66 93.0275) (width 0.381) (layer F.Cu) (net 5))
 (segment (start 122.2375 94.68) (end 122.2375 93.605) (width 0.381) (layer F.Cu) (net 5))
 (segment (start 121.66 93.0275) (end 120.3325 93.0275) (width 0.381) (layer F.Cu) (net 5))
 (segment (start 120.3325 93.0275) (end 119.6975 93.6625) (width 0.381) (layer F.Cu) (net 5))
 (segment (start 119.6975 93.6625) (end 119.6975 98.425) (width 0.381) (layer F.Cu) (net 5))
 (segment (start 119.6975 98.425) (end 118.745 99.3775) (width 0.381) (layer F.Cu) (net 5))
 (segment (start 118.745 99.3775) (end 110.8075 99.3775) (width 0.381) (layer F.Cu) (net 5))
 (segment (start 110.8075 99.3775) (end 110.8075 99.3775) (width 0.381) (layer F.Cu) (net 5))
 (via (at 110.8075 99.3775) (size 0.635) (drill 0.381) (layers F.Cu B.Cu) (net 5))
 (segment (start 110.8075 99.3775) (end 112.3225 99.3775) (width 0.381) (layer B.Cu) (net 5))
 (segment (start 123.1175 99.3775) (end 123.1175 101.6) (width 0.381) (layer B.Cu) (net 4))
 (segment (start 123.1175 101.6) (end 123.1175 102.625) (width 0.381) (layer B.Cu) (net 4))
 (segment (start 123.1175 102.625) (end 122.9525 102.79) (width 0.381) (layer B.Cu) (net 4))
 (segment (start 122.9525 102.79) (end 122.9525 104.4575) (width 0.381) (layer B.Cu) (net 4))
 (segment (start 121.8485 104.4575) (end 122.9525 104.4575) (width 0.381) (layer F.Cu) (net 4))
 (segment (start 120.9675 99.63) (end 120.9675 103.5765) (width 0.381) (layer F.Cu) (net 4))
 (segment (start 120.9675 103.5765) (end 121.8485 104.4575) (width 0.381) (layer F.Cu) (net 4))
 (via (at 123.5075 97.4725) (size 0.635) (drill 0.381) (layers F.Cu B.Cu) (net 10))
 (segment (start 123.190001 97.155001) (end 123.5075 97.4725) (width 0.381) (layer B.Cu) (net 10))
 (segment (start 122.2375 96.2025) (end 123.190001 97.155001) (width 0.381) (layer B.Cu) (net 10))
 (segment (start 122.2375 87.63) (end 122.2375 96.2025) (width 0.381) (layer B.Cu) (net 10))
 (segment (start 123.5075 99.63) (end 123.5075 97.4725) (width 0.381) (layer F.Cu) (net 10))
 (via (at 126.0475 97.4725) (size 0.635) (drill 0.381) (layers F.Cu B.Cu) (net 9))
 (segment (start 126.0475 99.63) (end 126.0475 97.4725) (width 0.381) (layer F.Cu) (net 9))
 (segment (start 124.7775 87.63) (end 124.7775 96.2025) (width 0.381) (layer B.Cu) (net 9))
 (segment (start 124.7775 96.2025) (end 125.730001 97.155001) (width 0.381) (layer B.Cu) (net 9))
 (segment (start 125.730001 97.155001) (end 126.0475 97.4725) (width 0.381) (layer B.Cu) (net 9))
 (segment (start 124.7775 93.127942) (end 124.7775 94.68) (width 0.381) (layer F.Cu) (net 7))
 (segment (start 127.3175 87.63) (end 127.3175 90.587942) (width 0.381) (layer F.Cu) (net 7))
 (segment (start 127.3175 90.587942) (end 124.7775 93.127942) (width 0.381) (layer F.Cu) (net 7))
 (via (at 128.5875 101.2825) (size 0.635) (drill 0.381) (layers F.Cu B.Cu) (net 1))
 (segment (start 133.9125 99.3775) (end 133.9125 101.6) (width 0.381) (layer B.Cu) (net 1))
 (segment (start 133.9125 101.6725) (end 133.9125 101.6) (width 0.254) (layer B.Cu) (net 1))
 (segment (start 133.6675 101.9175) (end 133.9125 101.6725) (width 0.254) (layer B.Cu) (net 1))
 (segment (start 133.7475 104.4575) (end 133.7475 101.9975) (width 0.381) (layer B.Cu) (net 1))
 (segment (start 133.7475 101.9975) (end 133.6675 101.9175) (width 0.254) (layer B.Cu) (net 1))
 (segment (start 133.9125 101.6) (end 129.8575 101.6) (width 0.381) (layer B.Cu) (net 1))
 (segment (start 129.54 101.2825) (end 128.5875 101.2825) (width 0.381) (layer B.Cu) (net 1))
 (segment (start 129.8575 101.6) (end 129.54 101.2825) (width 0.381) (layer B.Cu) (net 1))
 (segment (start 128.5875 99.63) (end 128.5875 101.2825) (width 0.381) (layer F.Cu) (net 1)))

